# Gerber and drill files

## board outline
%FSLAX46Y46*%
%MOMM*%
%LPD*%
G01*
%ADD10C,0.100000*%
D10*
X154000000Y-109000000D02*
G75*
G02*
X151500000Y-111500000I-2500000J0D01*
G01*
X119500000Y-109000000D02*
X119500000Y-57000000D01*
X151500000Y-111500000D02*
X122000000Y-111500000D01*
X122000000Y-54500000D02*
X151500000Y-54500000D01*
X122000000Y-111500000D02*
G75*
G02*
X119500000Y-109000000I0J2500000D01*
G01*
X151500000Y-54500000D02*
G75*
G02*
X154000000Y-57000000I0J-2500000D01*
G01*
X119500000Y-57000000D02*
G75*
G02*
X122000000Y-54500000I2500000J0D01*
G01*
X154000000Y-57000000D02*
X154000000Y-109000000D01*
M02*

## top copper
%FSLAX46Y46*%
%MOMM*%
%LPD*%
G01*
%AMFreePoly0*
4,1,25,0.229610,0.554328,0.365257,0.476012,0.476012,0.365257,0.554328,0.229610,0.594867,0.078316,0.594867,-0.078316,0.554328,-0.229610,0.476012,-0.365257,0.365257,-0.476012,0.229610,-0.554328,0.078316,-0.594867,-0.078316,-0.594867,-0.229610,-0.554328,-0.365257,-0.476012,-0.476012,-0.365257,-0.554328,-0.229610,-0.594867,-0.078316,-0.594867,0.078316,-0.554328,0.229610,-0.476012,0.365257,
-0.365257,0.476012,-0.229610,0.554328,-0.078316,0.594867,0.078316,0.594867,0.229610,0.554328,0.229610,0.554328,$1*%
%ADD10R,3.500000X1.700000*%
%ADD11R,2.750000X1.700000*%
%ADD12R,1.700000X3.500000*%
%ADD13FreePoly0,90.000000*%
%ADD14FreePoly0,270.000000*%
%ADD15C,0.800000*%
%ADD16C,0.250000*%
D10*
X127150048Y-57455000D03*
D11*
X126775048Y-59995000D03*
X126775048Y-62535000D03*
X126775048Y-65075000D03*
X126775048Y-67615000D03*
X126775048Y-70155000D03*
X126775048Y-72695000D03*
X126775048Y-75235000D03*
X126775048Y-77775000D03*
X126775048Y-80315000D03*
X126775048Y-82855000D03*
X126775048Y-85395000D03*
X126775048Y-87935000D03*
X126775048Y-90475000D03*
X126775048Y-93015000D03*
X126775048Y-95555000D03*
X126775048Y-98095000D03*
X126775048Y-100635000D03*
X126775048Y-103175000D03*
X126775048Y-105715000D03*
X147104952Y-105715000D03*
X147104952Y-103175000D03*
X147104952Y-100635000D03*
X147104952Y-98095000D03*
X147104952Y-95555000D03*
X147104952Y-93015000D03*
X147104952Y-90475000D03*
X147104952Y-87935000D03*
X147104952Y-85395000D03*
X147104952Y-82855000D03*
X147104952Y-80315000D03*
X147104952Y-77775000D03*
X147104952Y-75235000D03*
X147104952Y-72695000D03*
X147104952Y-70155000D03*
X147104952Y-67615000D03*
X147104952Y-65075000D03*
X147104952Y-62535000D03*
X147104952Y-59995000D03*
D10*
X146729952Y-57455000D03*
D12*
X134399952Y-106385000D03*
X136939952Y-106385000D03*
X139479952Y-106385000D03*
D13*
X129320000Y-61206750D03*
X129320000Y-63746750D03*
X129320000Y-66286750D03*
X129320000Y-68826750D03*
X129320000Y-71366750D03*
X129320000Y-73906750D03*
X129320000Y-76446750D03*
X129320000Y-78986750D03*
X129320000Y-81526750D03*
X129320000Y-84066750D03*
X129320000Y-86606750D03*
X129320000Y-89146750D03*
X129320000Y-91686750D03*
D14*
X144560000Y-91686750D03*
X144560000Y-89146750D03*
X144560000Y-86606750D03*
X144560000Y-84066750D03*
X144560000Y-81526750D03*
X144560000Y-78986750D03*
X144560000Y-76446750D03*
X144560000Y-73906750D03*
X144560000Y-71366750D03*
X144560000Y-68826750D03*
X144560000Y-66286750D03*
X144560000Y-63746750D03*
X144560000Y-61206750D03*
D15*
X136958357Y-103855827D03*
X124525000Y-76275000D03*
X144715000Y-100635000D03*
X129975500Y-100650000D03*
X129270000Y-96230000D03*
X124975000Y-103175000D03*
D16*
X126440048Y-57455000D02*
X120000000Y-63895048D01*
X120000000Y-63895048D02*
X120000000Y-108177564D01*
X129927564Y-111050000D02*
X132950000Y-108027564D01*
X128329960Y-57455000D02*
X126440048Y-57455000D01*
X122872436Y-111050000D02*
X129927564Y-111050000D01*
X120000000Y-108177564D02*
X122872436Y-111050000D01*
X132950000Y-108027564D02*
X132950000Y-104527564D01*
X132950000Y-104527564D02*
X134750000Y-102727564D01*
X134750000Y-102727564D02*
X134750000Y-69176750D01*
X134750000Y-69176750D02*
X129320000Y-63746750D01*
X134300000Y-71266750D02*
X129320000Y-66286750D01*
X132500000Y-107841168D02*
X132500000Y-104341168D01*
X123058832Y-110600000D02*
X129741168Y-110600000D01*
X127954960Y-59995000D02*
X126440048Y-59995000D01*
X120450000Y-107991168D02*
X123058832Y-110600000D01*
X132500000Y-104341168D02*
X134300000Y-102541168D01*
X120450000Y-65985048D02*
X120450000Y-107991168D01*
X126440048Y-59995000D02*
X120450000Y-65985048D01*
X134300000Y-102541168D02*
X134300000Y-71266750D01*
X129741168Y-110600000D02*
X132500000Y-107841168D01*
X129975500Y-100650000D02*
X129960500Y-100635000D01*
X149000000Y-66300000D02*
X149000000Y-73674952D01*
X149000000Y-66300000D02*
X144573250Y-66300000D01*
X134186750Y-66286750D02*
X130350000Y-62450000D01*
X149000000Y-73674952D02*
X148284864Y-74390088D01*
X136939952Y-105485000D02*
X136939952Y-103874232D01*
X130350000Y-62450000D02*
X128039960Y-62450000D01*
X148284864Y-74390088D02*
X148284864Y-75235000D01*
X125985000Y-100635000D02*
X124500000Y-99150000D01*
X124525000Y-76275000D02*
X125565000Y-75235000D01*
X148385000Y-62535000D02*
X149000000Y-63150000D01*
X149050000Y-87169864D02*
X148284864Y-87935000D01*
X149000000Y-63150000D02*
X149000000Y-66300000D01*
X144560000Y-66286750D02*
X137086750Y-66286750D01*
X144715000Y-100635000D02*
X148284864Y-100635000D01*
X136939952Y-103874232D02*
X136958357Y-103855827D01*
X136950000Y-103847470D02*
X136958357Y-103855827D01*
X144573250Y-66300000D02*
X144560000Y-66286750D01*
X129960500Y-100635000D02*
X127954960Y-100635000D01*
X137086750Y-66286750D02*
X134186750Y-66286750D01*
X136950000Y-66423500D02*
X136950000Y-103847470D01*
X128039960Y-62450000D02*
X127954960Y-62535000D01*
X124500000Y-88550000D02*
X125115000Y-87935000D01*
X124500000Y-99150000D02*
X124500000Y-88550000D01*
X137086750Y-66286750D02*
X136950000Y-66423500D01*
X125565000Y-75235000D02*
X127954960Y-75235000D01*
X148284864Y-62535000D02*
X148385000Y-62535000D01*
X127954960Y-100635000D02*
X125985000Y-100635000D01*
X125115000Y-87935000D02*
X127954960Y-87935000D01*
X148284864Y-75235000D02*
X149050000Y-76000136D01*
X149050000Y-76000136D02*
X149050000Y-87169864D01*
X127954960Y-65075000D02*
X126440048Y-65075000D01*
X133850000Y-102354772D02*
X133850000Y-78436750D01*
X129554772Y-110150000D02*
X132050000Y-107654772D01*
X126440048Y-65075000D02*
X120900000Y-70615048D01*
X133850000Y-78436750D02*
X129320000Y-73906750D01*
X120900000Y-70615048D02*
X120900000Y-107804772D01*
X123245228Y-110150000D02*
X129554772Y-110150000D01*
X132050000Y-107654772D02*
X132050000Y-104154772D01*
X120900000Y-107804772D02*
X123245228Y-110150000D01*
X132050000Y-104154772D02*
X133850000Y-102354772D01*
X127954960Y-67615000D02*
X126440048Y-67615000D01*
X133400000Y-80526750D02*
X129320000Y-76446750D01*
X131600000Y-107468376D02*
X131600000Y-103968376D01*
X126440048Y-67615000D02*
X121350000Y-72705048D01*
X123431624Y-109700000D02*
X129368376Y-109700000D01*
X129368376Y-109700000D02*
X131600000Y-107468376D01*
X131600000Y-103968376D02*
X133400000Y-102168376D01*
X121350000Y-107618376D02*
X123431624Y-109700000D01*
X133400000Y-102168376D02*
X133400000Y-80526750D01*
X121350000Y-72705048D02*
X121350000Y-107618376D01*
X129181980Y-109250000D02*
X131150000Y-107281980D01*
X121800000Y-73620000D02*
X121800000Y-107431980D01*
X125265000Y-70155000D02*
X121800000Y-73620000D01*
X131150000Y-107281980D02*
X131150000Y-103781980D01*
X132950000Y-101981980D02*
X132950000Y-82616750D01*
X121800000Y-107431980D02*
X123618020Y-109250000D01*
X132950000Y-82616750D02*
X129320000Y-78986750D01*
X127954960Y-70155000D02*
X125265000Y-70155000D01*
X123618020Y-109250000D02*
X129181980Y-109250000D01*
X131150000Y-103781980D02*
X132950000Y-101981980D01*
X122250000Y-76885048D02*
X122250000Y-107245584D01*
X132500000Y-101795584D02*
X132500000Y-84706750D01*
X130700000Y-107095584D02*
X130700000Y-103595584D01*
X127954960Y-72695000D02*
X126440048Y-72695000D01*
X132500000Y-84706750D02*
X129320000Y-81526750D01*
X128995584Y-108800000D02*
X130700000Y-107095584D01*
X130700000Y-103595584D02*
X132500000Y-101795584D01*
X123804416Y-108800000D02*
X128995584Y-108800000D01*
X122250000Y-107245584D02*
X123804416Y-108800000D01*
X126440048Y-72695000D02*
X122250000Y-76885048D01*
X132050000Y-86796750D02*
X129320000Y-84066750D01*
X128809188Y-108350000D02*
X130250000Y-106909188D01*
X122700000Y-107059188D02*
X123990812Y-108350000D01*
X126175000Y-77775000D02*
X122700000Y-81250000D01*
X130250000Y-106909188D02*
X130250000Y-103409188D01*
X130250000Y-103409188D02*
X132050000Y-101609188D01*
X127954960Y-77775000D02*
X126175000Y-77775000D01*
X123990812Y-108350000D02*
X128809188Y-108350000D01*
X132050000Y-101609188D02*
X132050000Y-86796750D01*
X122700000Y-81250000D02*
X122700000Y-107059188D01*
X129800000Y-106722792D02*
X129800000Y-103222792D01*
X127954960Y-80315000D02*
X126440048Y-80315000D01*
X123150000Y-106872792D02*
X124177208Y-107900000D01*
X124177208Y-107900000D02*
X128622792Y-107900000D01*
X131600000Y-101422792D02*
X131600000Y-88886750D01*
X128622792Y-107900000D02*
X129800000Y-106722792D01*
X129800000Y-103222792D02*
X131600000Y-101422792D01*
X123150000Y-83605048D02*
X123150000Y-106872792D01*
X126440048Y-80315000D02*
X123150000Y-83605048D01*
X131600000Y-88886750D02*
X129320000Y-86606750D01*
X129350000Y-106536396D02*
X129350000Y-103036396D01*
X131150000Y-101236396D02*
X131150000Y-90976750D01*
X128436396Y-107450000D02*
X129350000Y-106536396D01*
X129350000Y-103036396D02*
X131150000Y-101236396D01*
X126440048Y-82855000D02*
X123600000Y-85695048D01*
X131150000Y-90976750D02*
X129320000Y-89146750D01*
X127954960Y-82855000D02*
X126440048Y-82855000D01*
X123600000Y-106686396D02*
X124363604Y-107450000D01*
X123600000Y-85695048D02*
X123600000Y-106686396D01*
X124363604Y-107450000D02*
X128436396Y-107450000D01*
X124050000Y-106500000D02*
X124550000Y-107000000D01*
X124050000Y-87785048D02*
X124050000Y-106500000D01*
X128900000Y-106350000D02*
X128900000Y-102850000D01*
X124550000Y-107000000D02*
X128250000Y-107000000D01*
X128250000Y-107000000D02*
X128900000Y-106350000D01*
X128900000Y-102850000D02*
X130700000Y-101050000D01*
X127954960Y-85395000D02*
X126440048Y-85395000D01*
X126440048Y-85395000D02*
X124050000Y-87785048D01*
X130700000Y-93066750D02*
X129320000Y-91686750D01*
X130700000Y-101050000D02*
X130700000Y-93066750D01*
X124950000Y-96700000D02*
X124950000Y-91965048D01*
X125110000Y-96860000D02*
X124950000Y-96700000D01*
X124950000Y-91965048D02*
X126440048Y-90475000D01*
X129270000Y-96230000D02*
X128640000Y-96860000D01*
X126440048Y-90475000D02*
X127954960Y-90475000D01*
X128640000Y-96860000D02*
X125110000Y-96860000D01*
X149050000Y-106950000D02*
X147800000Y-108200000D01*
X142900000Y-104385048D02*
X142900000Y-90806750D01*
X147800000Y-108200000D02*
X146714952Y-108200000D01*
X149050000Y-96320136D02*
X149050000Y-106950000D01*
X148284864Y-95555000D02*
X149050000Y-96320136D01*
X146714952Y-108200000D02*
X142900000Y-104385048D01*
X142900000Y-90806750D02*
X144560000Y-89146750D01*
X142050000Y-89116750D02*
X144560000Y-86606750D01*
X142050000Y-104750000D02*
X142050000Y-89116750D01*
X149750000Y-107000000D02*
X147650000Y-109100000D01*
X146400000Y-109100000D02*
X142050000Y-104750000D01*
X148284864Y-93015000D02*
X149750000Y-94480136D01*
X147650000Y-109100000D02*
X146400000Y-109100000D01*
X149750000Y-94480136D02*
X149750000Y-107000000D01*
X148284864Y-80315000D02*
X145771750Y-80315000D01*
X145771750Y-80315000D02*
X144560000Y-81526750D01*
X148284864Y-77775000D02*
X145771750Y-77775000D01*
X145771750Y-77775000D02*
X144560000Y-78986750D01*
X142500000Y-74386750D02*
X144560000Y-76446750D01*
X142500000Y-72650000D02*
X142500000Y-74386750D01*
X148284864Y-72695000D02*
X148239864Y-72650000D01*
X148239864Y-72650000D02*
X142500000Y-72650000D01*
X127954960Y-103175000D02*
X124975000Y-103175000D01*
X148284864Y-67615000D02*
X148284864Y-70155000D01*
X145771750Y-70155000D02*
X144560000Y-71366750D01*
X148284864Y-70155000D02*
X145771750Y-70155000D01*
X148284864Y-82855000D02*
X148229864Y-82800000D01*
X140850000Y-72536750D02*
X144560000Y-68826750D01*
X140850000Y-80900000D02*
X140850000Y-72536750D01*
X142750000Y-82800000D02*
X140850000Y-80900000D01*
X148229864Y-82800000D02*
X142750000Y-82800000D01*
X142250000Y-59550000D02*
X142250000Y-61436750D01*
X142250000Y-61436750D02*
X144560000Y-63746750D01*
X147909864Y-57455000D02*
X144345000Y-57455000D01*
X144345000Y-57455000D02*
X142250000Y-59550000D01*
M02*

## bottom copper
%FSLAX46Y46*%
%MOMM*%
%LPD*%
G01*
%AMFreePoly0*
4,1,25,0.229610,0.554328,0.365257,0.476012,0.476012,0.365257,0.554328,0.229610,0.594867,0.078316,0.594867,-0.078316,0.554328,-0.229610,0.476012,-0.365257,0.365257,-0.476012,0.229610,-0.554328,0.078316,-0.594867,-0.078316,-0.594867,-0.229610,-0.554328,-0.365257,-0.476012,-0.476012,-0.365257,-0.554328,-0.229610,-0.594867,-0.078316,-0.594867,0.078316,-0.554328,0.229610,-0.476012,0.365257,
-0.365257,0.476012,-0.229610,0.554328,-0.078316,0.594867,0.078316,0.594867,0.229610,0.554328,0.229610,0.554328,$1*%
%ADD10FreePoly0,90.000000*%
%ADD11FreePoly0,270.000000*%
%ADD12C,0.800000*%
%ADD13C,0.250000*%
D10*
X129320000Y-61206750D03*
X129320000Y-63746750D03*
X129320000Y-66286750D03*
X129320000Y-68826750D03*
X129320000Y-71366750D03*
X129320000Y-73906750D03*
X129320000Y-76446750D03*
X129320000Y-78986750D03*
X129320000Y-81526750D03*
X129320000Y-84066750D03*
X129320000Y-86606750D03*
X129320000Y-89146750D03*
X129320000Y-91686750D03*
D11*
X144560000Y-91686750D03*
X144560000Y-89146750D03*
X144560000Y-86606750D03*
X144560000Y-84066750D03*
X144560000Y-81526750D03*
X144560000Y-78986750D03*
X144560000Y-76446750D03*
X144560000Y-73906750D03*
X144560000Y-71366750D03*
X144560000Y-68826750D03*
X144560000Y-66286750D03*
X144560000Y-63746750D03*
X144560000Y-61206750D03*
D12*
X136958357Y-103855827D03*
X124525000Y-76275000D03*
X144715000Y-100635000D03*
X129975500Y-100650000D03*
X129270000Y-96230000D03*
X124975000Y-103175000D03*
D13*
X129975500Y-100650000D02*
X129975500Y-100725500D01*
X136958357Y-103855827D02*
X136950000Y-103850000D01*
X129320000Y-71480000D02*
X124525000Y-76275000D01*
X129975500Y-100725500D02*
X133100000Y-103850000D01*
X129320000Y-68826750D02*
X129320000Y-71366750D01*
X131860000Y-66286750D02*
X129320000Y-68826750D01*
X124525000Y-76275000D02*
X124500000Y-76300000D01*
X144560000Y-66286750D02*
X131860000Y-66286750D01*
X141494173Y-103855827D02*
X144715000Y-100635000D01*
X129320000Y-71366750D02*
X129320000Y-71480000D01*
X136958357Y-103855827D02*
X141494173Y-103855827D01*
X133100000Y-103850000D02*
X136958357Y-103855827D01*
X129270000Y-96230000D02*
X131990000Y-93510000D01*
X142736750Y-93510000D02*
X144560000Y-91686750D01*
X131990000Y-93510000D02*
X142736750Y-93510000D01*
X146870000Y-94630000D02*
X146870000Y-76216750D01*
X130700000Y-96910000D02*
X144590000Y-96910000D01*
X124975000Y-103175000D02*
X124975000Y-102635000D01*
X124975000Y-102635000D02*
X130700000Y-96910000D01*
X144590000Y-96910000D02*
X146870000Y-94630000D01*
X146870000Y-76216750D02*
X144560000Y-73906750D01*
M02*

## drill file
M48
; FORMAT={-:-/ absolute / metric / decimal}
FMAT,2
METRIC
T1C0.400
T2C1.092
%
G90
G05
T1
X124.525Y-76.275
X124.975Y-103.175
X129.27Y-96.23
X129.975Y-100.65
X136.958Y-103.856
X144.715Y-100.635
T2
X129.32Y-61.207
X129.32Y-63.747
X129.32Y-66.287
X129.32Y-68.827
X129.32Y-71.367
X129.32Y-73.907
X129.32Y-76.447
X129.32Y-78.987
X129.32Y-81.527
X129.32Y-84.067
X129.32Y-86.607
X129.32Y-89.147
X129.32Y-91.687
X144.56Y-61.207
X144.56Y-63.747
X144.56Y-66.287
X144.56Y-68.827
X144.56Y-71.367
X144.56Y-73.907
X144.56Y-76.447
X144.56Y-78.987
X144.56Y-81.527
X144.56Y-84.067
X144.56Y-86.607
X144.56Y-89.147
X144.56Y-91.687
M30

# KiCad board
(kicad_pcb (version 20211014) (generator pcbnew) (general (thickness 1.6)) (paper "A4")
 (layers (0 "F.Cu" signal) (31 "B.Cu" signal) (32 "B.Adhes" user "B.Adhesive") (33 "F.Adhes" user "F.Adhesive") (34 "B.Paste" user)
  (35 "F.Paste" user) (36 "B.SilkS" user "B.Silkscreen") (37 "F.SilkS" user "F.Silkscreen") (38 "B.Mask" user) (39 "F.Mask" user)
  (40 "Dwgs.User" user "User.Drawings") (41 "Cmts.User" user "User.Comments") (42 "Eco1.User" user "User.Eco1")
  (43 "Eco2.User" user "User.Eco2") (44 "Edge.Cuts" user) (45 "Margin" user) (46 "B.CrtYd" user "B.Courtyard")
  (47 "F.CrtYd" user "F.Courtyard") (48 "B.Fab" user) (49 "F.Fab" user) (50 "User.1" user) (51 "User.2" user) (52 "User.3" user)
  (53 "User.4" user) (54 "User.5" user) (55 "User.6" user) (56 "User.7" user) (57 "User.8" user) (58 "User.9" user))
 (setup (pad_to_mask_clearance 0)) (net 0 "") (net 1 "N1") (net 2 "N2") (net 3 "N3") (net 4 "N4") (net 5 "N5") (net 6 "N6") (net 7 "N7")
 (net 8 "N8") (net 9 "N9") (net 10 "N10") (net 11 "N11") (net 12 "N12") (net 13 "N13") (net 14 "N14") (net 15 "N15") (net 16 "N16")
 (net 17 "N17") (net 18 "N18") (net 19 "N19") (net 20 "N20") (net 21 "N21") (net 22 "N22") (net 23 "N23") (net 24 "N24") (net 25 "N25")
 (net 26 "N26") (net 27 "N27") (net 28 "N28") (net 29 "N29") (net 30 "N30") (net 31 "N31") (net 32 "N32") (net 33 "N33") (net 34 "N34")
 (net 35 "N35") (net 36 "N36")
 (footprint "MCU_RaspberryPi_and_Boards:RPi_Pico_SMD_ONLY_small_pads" (layer "F.Cu") (at 136.939952 81.585)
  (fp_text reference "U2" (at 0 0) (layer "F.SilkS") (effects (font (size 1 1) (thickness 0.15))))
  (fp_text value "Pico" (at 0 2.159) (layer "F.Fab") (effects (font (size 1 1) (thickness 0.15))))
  (pad "1" smd rect (at -8.609992 -24.13) (size 3.5 1.7) (drill (offset -1.179912 0)) (layers "F.Cu" "F.Mask") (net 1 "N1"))
  (pad "2" smd rect (at -8.984992 -21.59) (size 2.75 1.7) (drill (offset -1.179912 0)) (layers "F.Cu" "F.Mask") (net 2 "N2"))
  (pad "3" smd rect (at -8.984992 -19.05) (size 2.75 1.7) (drill (offset -1.179912 0)) (layers "F.Cu" "F.Mask") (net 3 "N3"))
  (pad "4" smd rect (at -8.984992 -16.51) (size 2.75 1.7) (drill (offset -1.179912 0)) (layers "F.Cu" "F.Mask") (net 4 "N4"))
  (pad "5" smd rect (at -8.984992 -13.97) (size 2.75 1.7) (drill (offset -1.179912 0)) (layers "F.Cu" "F.Mask") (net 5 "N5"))
  (pad "6" smd rect (at -8.984992 -11.43) (size 2.75 1.7) (drill (offset -1.179912 0)) (layers "F.Cu" "F.Mask") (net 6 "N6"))
  (pad "7" smd rect (at -8.984992 -8.89) (size 2.75 1.7) (drill (offset -1.179912 0)) (layers "F.Cu" "F.Mask") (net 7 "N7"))
  (pad "8" smd rect (at -8.984992 -6.35) (size 2.75 1.7) (drill (offset -1.179912 0)) (layers "F.Cu" "F.Mask") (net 3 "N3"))
  (pad "9" smd rect (at -8.984992 -3.81) (size 2.75 1.7) (drill (offset -1.179912 0)) (layers "F.Cu" "F.Mask") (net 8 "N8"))
  (pad "10" smd rect (at -8.984992 -1.27) (size 2.75 1.7) (drill (offset -1.179912 0)) (layers "F.Cu" "F.Mask") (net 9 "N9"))
  (pad "11" smd rect (at -8.984992 1.27) (size 2.75 1.7) (drill (offset -1.179912 0)) (layers "F.Cu" "F.Mask") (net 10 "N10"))
  (pad "12" smd rect (at -8.984992 3.81) (size 2.75 1.7) (drill (offset -1.179912 0)) (layers "F.Cu" "F.Mask") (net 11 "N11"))
  (pad "13" smd rect (at -8.984992 6.35) (size 2.75 1.7) (drill (offset -1.179912 0)) (layers "F.Cu" "F.Mask") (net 3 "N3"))
  (pad "14" smd rect (at -8.984992 8.89) (size 2.75 1.7) (drill (offset -1.179912 0)) (layers "F.Cu" "F.Mask") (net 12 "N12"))
  (pad "15" smd rect (at -8.984992 11.43) (size 2.75 1.7) (drill (offset -1.179912 0)) (layers "F.Cu" "F.Mask") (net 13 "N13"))
  (pad "16" smd rect (at -8.984992 13.97) (size 2.75 1.7) (drill (offset -1.179912 0)) (layers "F.Cu" "F.Mask") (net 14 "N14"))
  (pad "17" smd rect (at -8.984992 16.51) (size 2.75 1.7) (drill (offset -1.179912 0)) (layers "F.Cu" "F.Mask") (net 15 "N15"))
  (pad "18" smd rect (at -8.984992 19.05) (size 2.75 1.7) (drill (offset -1.179912 0)) (layers "F.Cu" "F.Mask") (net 3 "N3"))
  (pad "19" smd rect (at -8.984992 21.59) (size 2.75 1.7) (drill (offset -1.179912 0)) (layers "F.Cu" "F.Mask") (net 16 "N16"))
  (pad "20" smd rect (at -8.984992 24.13) (size 2.75 1.7) (drill (offset -1.179912 0)) (layers "F.Cu" "F.Mask") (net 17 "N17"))
  (pad "21" smd rect (at 11.344912 24.13) (size 2.75 1.7) (drill (offset -1.179912 0)) (layers "F.Cu" "F.Mask") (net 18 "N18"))
  (pad "22" smd rect (at 11.344912 21.59) (size 2.75 1.7) (drill (offset -1.179912 0)) (layers "F.Cu" "F.Mask") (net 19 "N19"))
  (pad "23" smd rect (at 11.344912 19.05) (size 2.75 1.7) (drill (offset -1.179912 0)) (layers "F.Cu" "F.Mask") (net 3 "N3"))
  (pad "24" smd rect (at 11.344912 16.51) (size 2.75 1.7) (drill (offset -1.179912 0)) (layers "F.Cu" "F.Mask") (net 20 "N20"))
  (pad "25" smd rect (at 11.344912 13.97) (size 2.75 1.7) (drill (offset -1.179912 0)) (layers "F.Cu" "F.Mask") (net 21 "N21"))
  (pad "26" smd rect (at 11.344912 11.43) (size 2.75 1.7) (drill (offset -1.179912 0)) (layers "F.Cu" "F.Mask") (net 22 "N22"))
  (pad "27" smd rect (at 11.344912 8.89) (size 2.75 1.7) (drill (offset -1.179912 0)) (layers "F.Cu" "F.Mask") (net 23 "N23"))
  (pad "28" smd rect (at 11.344912 6.35) (size 2.75 1.7) (drill (offset -1.179912 0)) (layers "F.Cu" "F.Mask") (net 3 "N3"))
  (pad "29" smd rect (at 11.344912 3.81) (size 2.75 1.7) (drill (offset -1.179912 0)) (layers "F.Cu" "F.Mask") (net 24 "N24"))
  (pad "30" smd rect (at 11.344912 1.27) (size 2.75 1.7) (drill (offset -1.179912 0)) (layers "F.Cu" "F.Mask") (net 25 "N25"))
  (pad "31" smd rect (at 11.344912 -1.27) (size 2.75 1.7) (drill (offset -1.179912 0)) (layers "F.Cu" "F.Mask") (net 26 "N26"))
  (pad "32" smd rect (at 11.344912 -3.81) (size 2.75 1.7) (drill (offset -1.179912 0)) (layers "F.Cu" "F.Mask") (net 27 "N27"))
  (pad "33" smd rect (at 11.344912 -6.35) (size 2.75 1.7) (drill (offset -1.179912 0)) (layers "F.Cu" "F.Mask") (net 3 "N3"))
  (pad "34" smd rect (at 11.344912 -8.89) (size 2.75 1.7) (drill (offset -1.179912 0)) (layers "F.Cu" "F.Mask") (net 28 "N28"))
  (pad "35" smd rect (at 11.344912 -11.43) (size 2.75 1.7) (drill (offset -1.179912 0)) (layers "F.Cu" "F.Mask") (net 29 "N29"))
  (pad "36" smd rect (at 11.344912 -13.97) (size 2.75 1.7) (drill (offset -1.179912 0)) (layers "F.Cu" "F.Mask") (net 29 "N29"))
  (pad "37" smd rect (at 11.344912 -16.51) (size 2.75 1.7) (drill (offset -1.179912 0)) (layers "F.Cu" "F.Mask") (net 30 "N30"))
  (pad "38" smd rect (at 11.344912 -19.05) (size 2.75 1.7) (drill (offset -1.179912 0)) (layers "F.Cu" "F.Mask") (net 3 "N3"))
  (pad "39" smd rect (at 11.344912 -21.59) (size 2.75 1.7) (drill (offset -1.179912 0)) (layers "F.Cu" "F.Mask") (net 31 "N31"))
  (pad "40" smd rect (at 10.969912 -24.13) (size 3.5 1.7) (drill (offset -1.179912 0)) (layers "F.Cu" "F.Mask") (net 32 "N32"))
  (pad "41" smd rect (at -2.54 23.9 90) (size 3.5 1.7) (drill (offset -0.9 0)) (layers "F.Cu" "F.Mask") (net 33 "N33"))
  (pad "42" smd rect (at 0 23.9 90) (size 3.5 1.7) (drill (offset -0.9 0)) (layers "F.Cu" "F.Mask") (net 3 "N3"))
  (pad "43" smd rect (at 2.54 23.9 90) (size 3.5 1.7) (drill (offset -0.9 0)) (layers "F.Cu" "F.Mask") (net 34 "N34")))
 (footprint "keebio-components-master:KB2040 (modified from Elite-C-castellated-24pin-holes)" (layer "B.Cu") (at 136.94 77.71675 -90)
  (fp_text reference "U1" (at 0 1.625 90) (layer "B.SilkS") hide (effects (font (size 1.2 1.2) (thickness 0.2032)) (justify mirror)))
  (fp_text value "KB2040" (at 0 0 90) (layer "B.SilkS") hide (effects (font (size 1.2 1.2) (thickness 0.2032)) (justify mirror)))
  (pad "0" thru_hole custom (at -16.51 7.62 90) (size 1.2 1.2) (drill 1.0922) (layers *.Cu *.SilkS *.Mask) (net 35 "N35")
   (options (clearance outline) (anchor circle)) (primitives))
  (pad "1" thru_hole custom (at -13.97 7.62 90) (size 1.2 1.2) (drill 1.0922) (layers *.Cu *.SilkS *.Mask) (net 1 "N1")
   (options (clearance outline) (anchor circle)) (primitives))
  (pad "2" thru_hole custom (at -11.43 7.62 90) (size 1.2 1.2) (drill 1.0922) (layers *.Cu *.SilkS *.Mask) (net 2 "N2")
   (options (clearance outline) (anchor circle)) (primitives))
  (pad "3" thru_hole custom (at -8.89 7.62 90) (size 1.2 1.2) (drill 1.0922) (layers *.Cu *.SilkS *.Mask) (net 3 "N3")
   (options (clearance outline) (anchor circle)) (primitives))
  (pad "4" thru_hole custom (at -6.35 7.62 90) (size 1.2 1.2) (drill 1.0922) (layers *.Cu *.SilkS *.Mask) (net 3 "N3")
   (options (clearance outline) (anchor circle)) (primitives))
  (pad "5" thru_hole custom (at -3.81 7.62 90) (size 1.2 1.2) (drill 1.0922) (layers *.Cu *.SilkS *.Mask) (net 4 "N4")
   (options (clearance outline) (anchor circle)) (primitives))
  (pad "6" thru_hole custom (at -1.27 7.62 90) (size 1.2 1.2) (drill 1.0922) (layers *.Cu *.SilkS *.Mask) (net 5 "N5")
   (options (clearance outline) (anchor circle)) (primitives))
  (pad "7" thru_hole custom (at 1.27 7.62 90) (size 1.2 1.2) (drill 1.0922) (layers *.Cu *.SilkS *.Mask) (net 6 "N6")
   (options (clearance outline) (anchor circle)) (primitives))
  (pad "8" thru_hole custom (at 3.81 7.62 90) (size 1.2 1.2) (drill 1.0922) (layers *.Cu *.SilkS *.Mask) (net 7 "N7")
   (options (clearance outline) (anchor circle)) (primitives))
  (pad "9" thru_hole custom (at 6.35 7.62 90) (size 1.2 1.2) (drill 1.0922) (layers *.Cu *.SilkS *.Mask) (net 8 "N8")
   (options (clearance outline) (anchor circle)) (primitives))
  (pad "10" thru_hole custom (at 8.89 7.62 90) (size 1.2 1.2) (drill 1.0922) (layers *.Cu *.SilkS *.Mask) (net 9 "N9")
   (options (clearance outline) (anchor circle)) (primitives))
  (pad "11" thru_hole custom (at 11.43 7.62 90) (size 1.2 1.2) (drill 1.0922) (layers *.Cu *.SilkS *.Mask) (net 10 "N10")
   (options (clearance outline) (anchor circle)) (primitives))
  (pad "12" thru_hole custom (at 13.97 7.62 90) (size 1.2 1.2) (drill 1.0922) (layers *.Cu *.SilkS *.Mask) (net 11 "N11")
   (options (clearance outline) (anchor circle)) (primitives))
  (pad "13" thru_hole custom (at 13.97 -7.62 270) (size 1.2 1.2) (drill 1.0922) (layers *.Cu *.SilkS *.Mask) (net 12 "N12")
   (options (clearance outline) (anchor circle)) (primitives))
  (pad "14" thru_hole custom (at 11.43 -7.62 270) (size 1.2 1.2) (drill 1.0922) (layers *.Cu *.SilkS *.Mask) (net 21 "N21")
   (options (clearance outline) (anchor circle)) (primitives))
  (pad "15" thru_hole custom (at 8.89 -7.62 270) (size 1.2 1.2) (drill 1.0922) (layers *.Cu *.SilkS *.Mask) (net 22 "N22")
   (options (clearance outline) (anchor circle)) (primitives))
  (pad "16" thru_hole custom (at 6.35 -7.62 270) (size 1.2 1.2) (drill 1.0922) (layers *.Cu *.SilkS *.Mask) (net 20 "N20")
   (options (clearance outline) (anchor circle)) (primitives))
  (pad "17" thru_hole custom (at 3.81 -7.62 270) (size 1.2 1.2) (drill 1.0922) (layers *.Cu *.SilkS *.Mask) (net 26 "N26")
   (options (clearance outline) (anchor circle)) (primitives))
  (pad "18" thru_hole custom (at 1.27 -7.62 270) (size 1.2 1.2) (drill 1.0922) (layers *.Cu *.SilkS *.Mask) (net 27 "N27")
   (options (clearance outline) (anchor circle)) (primitives))
  (pad "19" thru_hole custom (at -1.27 -7.62 270) (size 1.2 1.2) (drill 1.0922) (layers *.Cu *.SilkS *.Mask) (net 28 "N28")
   (options (clearance outline) (anchor circle)) (primitives))
  (pad "20" thru_hole custom (at -3.81 -7.62 270) (size 1.2 1.2) (drill 1.0922) (layers *.Cu *.SilkS *.Mask) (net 16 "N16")
   (options (clearance outline) (anchor circle)) (primitives))
  (pad "21" thru_hole custom (at -6.35 -7.62 270) (size 1.2 1.2) (drill 1.0922) (layers *.Cu *.SilkS *.Mask) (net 29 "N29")
   (options (clearance outline) (anchor circle)) (primitives))
  (pad "22" thru_hole custom (at -8.89 -7.62 270) (size 1.2 1.2) (drill 1.0922) (layers *.Cu *.SilkS *.Mask) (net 25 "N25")
   (options (clearance outline) (anchor circle)) (primitives))
  (pad "23" thru_hole custom (at -11.43 -7.62 270) (size 1.2 1.2) (drill 1.0922) (layers *.Cu *.SilkS *.Mask) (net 3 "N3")
   (options (clearance outline) (anchor circle)) (primitives))
  (pad "24" thru_hole custom (at -13.97 -7.62 270) (size 1.2 1.2) (drill 1.0922) (layers *.Cu *.SilkS *.Mask) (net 32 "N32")
   (options (clearance outline) (anchor circle)) (primitives))
  (pad "25" thru_hole custom (at -16.51 -7.62 270) (size 1.2 1.2) (drill 1.0922) (layers *.Cu *.SilkS *.Mask) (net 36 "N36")
   (options (clearance outline) (anchor circle)) (primitives)))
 (gr_arc (start 154 109) (mid 153.267767 110.767767) (end 151.5 111.5) (layer "Edge.Cuts") (width 0.1))
 (gr_line (start 119.5 109) (end 119.5 57) (layer "Edge.Cuts") (width 0.1))
 (gr_line (start 151.5 111.5) (end 122 111.5) (layer "Edge.Cuts") (width 0.1))
 (gr_line (start 122 54.5) (end 151.5 54.5) (layer "Edge.Cuts") (width 0.1))
 (gr_arc (start 122 111.5) (mid 120.232233 110.767767) (end 119.5 109) (layer "Edge.Cuts") (width 0.1))
 (gr_arc (start 151.5 54.5) (mid 153.267767 55.232233) (end 154 57) (layer "Edge.Cuts") (width 0.1))
 (gr_arc (start 119.5 57) (mid 120.232233 55.232233) (end 122 54.5) (layer "Edge.Cuts") (width 0.1))
 (gr_line (start 154 57) (end 154 109) (layer "Edge.Cuts") (width 0.1))
 (segment (start 126.440048 57.455) (end 120 63.895048) (width 0.25) (layer "F.Cu") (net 1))
 (segment (start 120 63.895048) (end 120 108.177564) (width 0.25) (layer "F.Cu") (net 1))
 (segment (start 129.927564 111.05) (end 132.95 108.027564) (width 0.25) (layer "F.Cu") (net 1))
 (segment (start 128.32996 57.455) (end 126.440048 57.455) (width 0.25) (layer "F.Cu") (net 1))
 (segment (start 122.872436 111.05) (end 129.927564 111.05) (width 0.25) (layer "F.Cu") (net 1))
 (segment (start 120 108.177564) (end 122.872436 111.05) (width 0.25) (layer "F.Cu") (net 1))
 (segment (start 132.95 108.027564) (end 132.95 104.527564) (width 0.25) (layer "F.Cu") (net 1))
 (segment (start 132.95 104.527564) (end 134.75 102.727564) (width 0.25) (layer "F.Cu") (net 1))
 (segment (start 134.75 102.727564) (end 134.75 69.17675) (width 0.25) (layer "F.Cu") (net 1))
 (segment (start 134.75 69.17675) (end 129.32 63.74675) (width 0.25) (layer "F.Cu") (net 1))
 (segment (start 134.3 71.26675) (end 129.32 66.28675) (width 0.25) (layer "F.Cu") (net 2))
 (segment (start 132.5 107.841168) (end 132.5 104.341168) (width 0.25) (layer "F.Cu") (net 2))
 (segment (start 123.058832 110.6) (end 129.741168 110.6) (width 0.25) (layer "F.Cu") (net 2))
 (segment (start 127.95496 59.995) (end 126.440048 59.995) (width 0.25) (layer "F.Cu") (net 2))
 (segment (start 120.45 107.991168) (end 123.058832 110.6) (width 0.25) (layer "F.Cu") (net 2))
 (segment (start 132.5 104.341168) (end 134.3 102.541168) (width 0.25) (layer "F.Cu") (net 2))
 (segment (start 120.45 65.985048) (end 120.45 107.991168) (width 0.25) (layer "F.Cu") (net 2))
 (segment (start 126.440048 59.995) (end 120.45 65.985048) (width 0.25) (layer "F.Cu") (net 2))
 (segment (start 134.3 102.541168) (end 134.3 71.26675) (width 0.25) (layer "F.Cu") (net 2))
 (segment (start 129.741168 110.6) (end 132.5 107.841168) (width 0.25) (layer "F.Cu") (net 2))
 (segment (start 129.9755 100.65) (end 129.9605 100.635) (width 0.25) (layer "F.Cu") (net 3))
 (segment (start 149 66.3) (end 149 73.674952) (width 0.25) (layer "F.Cu") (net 3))
 (segment (start 149 66.3) (end 144.57325 66.3) (width 0.25) (layer "F.Cu") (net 3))
 (segment (start 134.18675 66.28675) (end 130.35 62.45) (width 0.25) (layer "F.Cu") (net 3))
 (segment (start 149 73.674952) (end 148.284864 74.390088) (width 0.25) (layer "F.Cu") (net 3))
 (segment (start 136.939952 105.485) (end 136.939952 103.874232) (width 0.25) (layer "F.Cu") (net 3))
 (segment (start 130.35 62.45) (end 128.03996 62.45) (width 0.25) (layer "F.Cu") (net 3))
 (segment (start 148.284864 74.390088) (end 148.284864 75.235) (width 0.25) (layer "F.Cu") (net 3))
 (segment (start 125.985 100.635) (end 124.5 99.15) (width 0.25) (layer "F.Cu") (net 3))
 (segment (start 124.525 76.275) (end 125.565 75.235) (width 0.25) (layer "F.Cu") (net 3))
 (segment (start 148.385 62.535) (end 149 63.15) (width 0.25) (layer "F.Cu") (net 3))
 (segment (start 149.05 87.169864) (end 148.284864 87.935) (width 0.25) (layer "F.Cu") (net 3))
 (segment (start 149 63.15) (end 149 66.3) (width 0.25) (layer "F.Cu") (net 3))
 (segment (start 144.56 66.28675) (end 137.08675 66.28675) (width 0.25) (layer "F.Cu") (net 3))
 (segment (start 144.715 100.635) (end 148.284864 100.635) (width 0.25) (layer "F.Cu") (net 3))
 (segment (start 136.939952 103.874232) (end 136.958357 103.855827) (width 0.25) (layer "F.Cu") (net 3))
 (segment (start 136.95 103.84747) (end 136.958357 103.855827) (width 0.25) (layer "F.Cu") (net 3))
 (segment (start 144.57325 66.3) (end 144.56 66.28675) (width 0.25) (layer "F.Cu") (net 3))
 (segment (start 129.9605 100.635) (end 127.95496 100.635) (width 0.25) (layer "F.Cu") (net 3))
 (segment (start 137.08675 66.28675) (end 134.18675 66.28675) (width 0.25) (layer "F.Cu") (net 3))
 (segment (start 136.95 66.4235) (end 136.95 103.84747) (width 0.25) (layer "F.Cu") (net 3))
 (segment (start 128.03996 62.45) (end 127.95496 62.535) (width 0.25) (layer "F.Cu") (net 3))
 (segment (start 124.5 88.55) (end 125.115 87.935) (width 0.25) (layer "F.Cu") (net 3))
 (segment (start 124.5 99.15) (end 124.5 88.55) (width 0.25) (layer "F.Cu") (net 3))
 (segment (start 137.08675 66.28675) (end 136.95 66.4235) (width 0.25) (layer "F.Cu") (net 3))
 (segment (start 125.565 75.235) (end 127.95496 75.235) (width 0.25) (layer "F.Cu") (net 3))
 (segment (start 148.284864 62.535) (end 148.385 62.535) (width 0.25) (layer "F.Cu") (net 3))
 (segment (start 127.95496 100.635) (end 125.985 100.635) (width 0.25) (layer "F.Cu") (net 3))
 (segment (start 125.115 87.935) (end 127.95496 87.935) (width 0.25) (layer "F.Cu") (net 3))
 (segment (start 148.284864 75.235) (end 149.05 76.000136) (width 0.25) (layer "F.Cu") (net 3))
 (segment (start 149.05 76.000136) (end 149.05 87.169864) (width 0.25) (layer "F.Cu") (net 3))
 (via (at 136.958357 103.855827) (size 0.8) (drill 0.4) (layers "F.Cu" "B.Cu") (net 3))
 (via (at 124.525 76.275) (size 0.8) (drill 0.4) (layers "F.Cu" "B.Cu") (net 3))
 (via (at 144.715 100.635) (size 0.8) (drill 0.4) (layers "F.Cu" "B.Cu") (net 3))
 (via (at 129.9755 100.65) (size 0.8) (drill 0.4) (layers "F.Cu" "B.Cu") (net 3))
 (segment (start 129.9755 100.65) (end 129.9755 100.7255) (width 0.25) (layer "B.Cu") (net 3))
 (segment (start 136.958357 103.855827) (end 136.95 103.85) (width 0.25) (layer "B.Cu") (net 3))
 (segment (start 129.32 71.48) (end 124.525 76.275) (width 0.25) (layer "B.Cu") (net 3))
 (segment (start 129.9755 100.7255) (end 133.1 103.85) (width 0.25) (layer "B.Cu") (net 3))
 (segment (start 129.32 68.82675) (end 129.32 71.36675) (width 0.25) (layer "B.Cu") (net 3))
 (segment (start 131.86 66.28675) (end 129.32 68.82675) (width 0.25) (layer "B.Cu") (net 3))
 (segment (start 124.525 76.275) (end 124.5 76.3) (width 0.25) (layer "B.Cu") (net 3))
 (segment (start 144.56 66.28675) (end 131.86 66.28675) (width 0.25) (layer "B.Cu") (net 3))
 (segment (start 141.494173 103.855827) (end 144.715 100.635) (width 0.25) (layer "B.Cu") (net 3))
 (segment (start 129.32 71.36675) (end 129.32 71.48) (width 0.25) (layer "B.Cu") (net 3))
 (segment (start 136.958357 103.855827) (end 141.494173 103.855827) (width 0.25) (layer "B.Cu") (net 3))
 (segment (start 133.1 103.85) (end 136.958357 103.855827) (width 0.25) (layer "B.Cu") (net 3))
 (segment (start 127.95496 65.075) (end 126.440048 65.075) (width 0.25) (layer "F.Cu") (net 4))
 (segment (start 133.85 102.354772) (end 133.85 78.43675) (width 0.25) (layer "F.Cu") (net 4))
 (segment (start 129.554772 110.15) (end 132.05 107.654772) (width 0.25) (layer "F.Cu") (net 4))
 (segment (start 126.440048 65.075) (end 120.9 70.615048) (width 0.25) (layer "F.Cu") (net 4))
 (segment (start 133.85 78.43675) (end 129.32 73.90675) (width 0.25) (layer "F.Cu") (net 4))
 (segment (start 120.9 70.615048) (end 120.9 107.804772) (width 0.25) (layer "F.Cu") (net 4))
 (segment (start 123.245228 110.15) (end 129.554772 110.15) (width 0.25) (layer "F.Cu") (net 4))
 (segment (start 132.05 107.654772) (end 132.05 104.154772) (width 0.25) (layer "F.Cu") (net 4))
 (segment (start 120.9 107.804772) (end 123.245228 110.15) (width 0.25) (layer "F.Cu") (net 4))
 (segment (start 132.05 104.154772) (end 133.85 102.354772) (width 0.25) (layer "F.Cu") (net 4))
 (segment (start 127.95496 67.615) (end 126.440048 67.615) (width 0.25) (layer "F.Cu") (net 5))
 (segment (start 133.4 80.52675) (end 129.32 76.44675) (width 0.25) (layer "F.Cu") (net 5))
 (segment (start 131.6 107.468376) (end 131.6 103.968376) (width 0.25) (layer "F.Cu") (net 5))
 (segment (start 126.440048 67.615) (end 121.35 72.705048) (width 0.25) (layer "F.Cu") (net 5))
 (segment (start 123.431624 109.7) (end 129.368376 109.7) (width 0.25) (layer "F.Cu") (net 5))
 (segment (start 129.368376 109.7) (end 131.6 107.468376) (width 0.25) (layer "F.Cu") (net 5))
 (segment (start 131.6 103.968376) (end 133.4 102.168376) (width 0.25) (layer "F.Cu") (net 5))
 (segment (start 121.35 107.618376) (end 123.431624 109.7) (width 0.25) (layer "F.Cu") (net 5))
 (segment (start 133.4 102.168376) (end 133.4 80.52675) (width 0.25) (layer "F.Cu") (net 5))
 (segment (start 121.35 72.705048) (end 121.35 107.618376) (width 0.25) (layer "F.Cu") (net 5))
 (segment (start 129.18198 109.25) (end 131.15 107.28198) (width 0.25) (layer "F.Cu") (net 6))
 (segment (start 121.8 73.62) (end 121.8 107.43198) (width 0.25) (layer "F.Cu") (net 6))
 (segment (start 125.265 70.155) (end 121.8 73.62) (width 0.25) (layer "F.Cu") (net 6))
 (segment (start 131.15 107.28198) (end 131.15 103.78198) (width 0.25) (layer "F.Cu") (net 6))
 (segment (start 132.95 101.98198) (end 132.95 82.61675) (width 0.25) (layer "F.Cu") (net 6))
 (segment (start 121.8 107.43198) (end 123.61802 109.25) (width 0.25) (layer "F.Cu") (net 6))
 (segment (start 132.95 82.61675) (end 129.32 78.98675) (width 0.25) (layer "F.Cu") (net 6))
 (segment (start 127.95496 70.155) (end 125.265 70.155) (width 0.25) (layer "F.Cu") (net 6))
 (segment (start 123.61802 109.25) (end 129.18198 109.25) (width 0.25) (layer "F.Cu") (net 6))
 (segment (start 131.15 103.78198) (end 132.95 101.98198) (width 0.25) (layer "F.Cu") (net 6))
 (segment (start 122.25 76.885048) (end 122.25 107.245584) (width 0.25) (layer "F.Cu") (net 7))
 (segment (start 132.5 101.795584) (end 132.5 84.70675) (width 0.25) (layer "F.Cu") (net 7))
 (segment (start 130.7 107.095584) (end 130.7 103.595584) (width 0.25) (layer "F.Cu") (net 7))
 (segment (start 127.95496 72.695) (end 126.440048 72.695) (width 0.25) (layer "F.Cu") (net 7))
 (segment (start 132.5 84.70675) (end 129.32 81.52675) (width 0.25) (layer "F.Cu") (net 7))
 (segment (start 128.995584 108.8) (end 130.7 107.095584) (width 0.25) (layer "F.Cu") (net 7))
 (segment (start 130.7 103.595584) (end 132.5 101.795584) (width 0.25) (layer "F.Cu") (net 7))
 (segment (start 123.804416 108.8) (end 128.995584 108.8) (width 0.25) (layer "F.Cu") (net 7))
 (segment (start 122.25 107.245584) (end 123.804416 108.8) (width 0.25) (layer "F.Cu") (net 7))
 (segment (start 126.440048 72.695) (end 122.25 76.885048) (width 0.25) (layer "F.Cu") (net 7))
 (segment (start 132.05 86.79675) (end 129.32 84.06675) (width 0.25) (layer "F.Cu") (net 8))
 (segment (start 128.809188 108.35) (end 130.25 106.909188) (width 0.25) (layer "F.Cu") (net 8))
 (segment (start 122.7 107.059188) (end 123.990812 108.35) (width 0.25) (layer "F.Cu") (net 8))
 (segment (start 126.175 77.775) (end 122.7 81.25) (width 0.25) (layer "F.Cu") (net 8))
 (segment (start 130.25 106.909188) (end 130.25 103.409188) (width 0.25) (layer "F.Cu") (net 8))
 (segment (start 130.25 103.409188) (end 132.05 101.609188) (width 0.25) (layer "F.Cu") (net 8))
 (segment (start 127.95496 77.775) (end 126.175 77.775) (width 0.25) (layer "F.Cu") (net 8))
 (segment (start 123.990812 108.35) (end 128.809188 108.35) (width 0.25) (layer "F.Cu") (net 8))
 (segment (start 132.05 101.609188) (end 132.05 86.79675) (width 0.25) (layer "F.Cu") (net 8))
 (segment (start 122.7 81.25) (end 122.7 107.059188) (width 0.25) (layer "F.Cu") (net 8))
 (segment (start 129.8 106.722792) (end 129.8 103.222792) (width 0.25) (layer "F.Cu") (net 9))
 (segment (start 127.95496 80.315) (end 126.440048 80.315) (width 0.25) (layer "F.Cu") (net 9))
 (segment (start 123.15 106.872792) (end 124.177208 107.9) (width 0.25) (layer "F.Cu") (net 9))
 (segment (start 124.177208 107.9) (end 128.622792 107.9) (width 0.25) (layer "F.Cu") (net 9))
 (segment (start 131.6 101.422792) (end 131.6 88.88675) (width 0.25) (layer "F.Cu") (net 9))
 (segment (start 128.622792 107.9) (end 129.8 106.722792) (width 0.25) (layer "F.Cu") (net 9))
 (segment (start 129.8 103.222792) (end 131.6 101.422792) (width 0.25) (layer "F.Cu") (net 9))
 (segment (start 123.15 83.605048) (end 123.15 106.872792) (width 0.25) (layer "F.Cu") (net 9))
 (segment (start 126.440048 80.315) (end 123.15 83.605048) (width 0.25) (layer "F.Cu") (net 9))
 (segment (start 131.6 88.88675) (end 129.32 86.60675) (width 0.25) (layer "F.Cu") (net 9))
 (segment (start 129.35 106.536396) (end 129.35 103.036396) (width 0.25) (layer "F.Cu") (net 10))
 (segment (start 131.15 101.236396) (end 131.15 90.97675) (width 0.25) (layer "F.Cu") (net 10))
 (segment (start 128.436396 107.45) (end 129.35 106.536396) (width 0.25) (layer "F.Cu") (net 10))
 (segment (start 129.35 103.036396) (end 131.15 101.236396) (width 0.25) (layer "F.Cu") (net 10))
 (segment (start 126.440048 82.855) (end 123.6 85.695048) (width 0.25) (layer "F.Cu") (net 10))
 (segment (start 131.15 90.97675) (end 129.32 89.14675) (width 0.25) (layer "F.Cu") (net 10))
 (segment (start 127.95496 82.855) (end 126.440048 82.855) (width 0.25) (layer "F.Cu") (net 10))
 (segment (start 123.6 106.686396) (end 124.363604 107.45) (width 0.25) (layer "F.Cu") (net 10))
 (segment (start 123.6 85.695048) (end 123.6 106.686396) (width 0.25) (layer "F.Cu") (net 10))
 (segment (start 124.363604 107.45) (end 128.436396 107.45) (width 0.25) (layer "F.Cu") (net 10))
 (segment (start 124.05 106.5) (end 124.55 107) (width 0.25) (layer "F.Cu") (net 11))
 (segment (start 124.05 87.785048) (end 124.05 106.5) (width 0.25) (layer "F.Cu") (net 11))
 (segment (start 128.9 106.35) (end 128.9 102.85) (width 0.25) (layer "F.Cu") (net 11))
 (segment (start 124.55 107) (end 128.25 107) (width 0.25) (layer "F.Cu") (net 11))
 (segment (start 128.25 107) (end 128.9 106.35) (width 0.25) (layer "F.Cu") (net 11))
 (segment (start 128.9 102.85) (end 130.7 101.05) (width 0.25) (layer "F.Cu") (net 11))
 (segment (start 127.95496 85.395) (end 126.440048 85.395) (width 0.25) (layer "F.Cu") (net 11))
 (segment (start 126.440048 85.395) (end 124.05 87.785048) (width 0.25) (layer "F.Cu") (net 11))
 (segment (start 130.7 93.06675) (end 129.32 91.68675) (width 0.25) (layer "F.Cu") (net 11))
 (segment (start 130.7 101.05) (end 130.7 93.06675) (width 0.25) (layer "F.Cu") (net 11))
 (segment (start 124.95 96.7) (end 124.95 91.965048) (width 0.25) (layer "F.Cu") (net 12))
 (segment (start 125.11 96.86) (end 124.95 96.7) (width 0.25) (layer "F.Cu") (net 12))
 (segment (start 124.95 91.965048) (end 126.440048 90.475) (width 0.25) (layer "F.Cu") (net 12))
 (segment (start 129.27 96.23) (end 128.64 96.86) (width 0.25) (layer "F.Cu") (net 12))
 (segment (start 126.440048 90.475) (end 127.95496 90.475) (width 0.25) (layer "F.Cu") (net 12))
 (segment (start 128.64 96.86) (end 125.11 96.86) (width 0.25) (layer "F.Cu") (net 12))
 (via (at 129.27 96.23) (size 0.8) (drill 0.4) (layers "F.Cu" "B.Cu") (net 12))
 (segment (start 129.27 96.23) (end 131.99 93.51) (width 0.25) (layer "B.Cu") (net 12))
 (segment (start 142.73675 93.51) (end 144.56 91.68675) (width 0.25) (layer "B.Cu") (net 12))
 (segment (start 131.99 93.51) (end 142.73675 93.51) (width 0.25) (layer "B.Cu") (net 12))
 (segment (start 149.05 106.95) (end 147.8 108.2) (width 0.25) (layer "F.Cu") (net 21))
 (segment (start 142.9 104.385048) (end 142.9 90.80675) (width 0.25) (layer "F.Cu") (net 21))
 (segment (start 147.8 108.2) (end 146.714952 108.2) (width 0.25) (layer "F.Cu") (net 21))
 (segment (start 149.05 96.320136) (end 149.05 106.95) (width 0.25) (layer "F.Cu") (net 21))
 (segment (start 148.284864 95.555) (end 149.05 96.320136) (width 0.25) (layer "F.Cu") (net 21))
 (segment (start 146.714952 108.2) (end 142.9 104.385048) (width 0.25) (layer "F.Cu") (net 21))
 (segment (start 142.9 90.80675) (end 144.56 89.14675) (width 0.25) (layer "F.Cu") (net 21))
 (segment (start 142.05 89.11675) (end 144.56 86.60675) (width 0.25) (layer "F.Cu") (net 22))
 (segment (start 142.05 104.75) (end 142.05 89.11675) (width 0.25) (layer "F.Cu") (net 22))
 (segment (start 149.75 107) (end 147.65 109.1) (width 0.25) (layer "F.Cu") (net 22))
 (segment (start 146.4 109.1) (end 142.05 104.75) (width 0.25) (layer "F.Cu") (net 22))
 (segment (start 148.284864 93.015) (end 149.75 94.480136) (width 0.25) (layer "F.Cu") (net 22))
 (segment (start 147.65 109.1) (end 146.4 109.1) (width 0.25) (layer "F.Cu") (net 22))
 (segment (start 149.75 94.480136) (end 149.75 107) (width 0.25) (layer "F.Cu") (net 22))
 (segment (start 148.284864 80.315) (end 145.77175 80.315) (width 0.25) (layer "F.Cu") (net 26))
 (segment (start 145.77175 80.315) (end 144.56 81.52675) (width 0.25) (layer "F.Cu") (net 26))
 (segment (start 148.284864 77.775) (end 145.77175 77.775) (width 0.25) (layer "F.Cu") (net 27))
 (segment (start 145.77175 77.775) (end 144.56 78.98675) (width 0.25) (layer "F.Cu") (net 27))
 (segment (start 142.5 74.38675) (end 144.56 76.44675) (width 0.25) (layer "F.Cu") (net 28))
 (segment (start 142.5 72.65) (end 142.5 74.38675) (width 0.25) (layer "F.Cu") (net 28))
 (segment (start 148.284864 72.695) (end 148.239864 72.65) (width 0.25) (layer "F.Cu") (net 28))
 (segment (start 148.239864 72.65) (end 142.5 72.65) (width 0.25) (layer "F.Cu") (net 28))
 (segment (start 127.95496 103.175) (end 124.975 103.175) (width 0.25) (layer "F.Cu") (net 16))
 (via (at 124.975 103.175) (size 0.8) (drill 0.4) (layers "F.Cu" "B.Cu") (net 16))
 (segment (start 146.87 94.63) (end 146.87 76.21675) (width 0.25) (layer "B.Cu") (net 16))
 (segment (start 130.7 96.91) (end 144.59 96.91) (width 0.25) (layer "B.Cu") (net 16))
 (segment (start 124.975 103.175) (end 124.975 102.635) (width 0.25) (layer "B.Cu") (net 16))
 (segment (start 124.975 102.635) (end 130.7 96.91) (width 0.25) (layer "B.Cu") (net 16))
 (segment (start 144.59 96.91) (end 146.87 94.63) (width 0.25) (layer "B.Cu") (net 16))
 (segment (start 146.87 76.21675) (end 144.56 73.90675) (width 0.25) (layer "B.Cu") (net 16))
 (segment (start 148.284864 67.615) (end 148.284864 70.155) (width 0.25) (layer "F.Cu") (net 29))
 (segment (start 145.77175 70.155) (end 144.56 71.36675) (width 0.25) (layer "F.Cu") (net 29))
 (segment (start 148.284864 70.155) (end 145.77175 70.155) (width 0.25) (layer "F.Cu") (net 29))
 (segment (start 148.284864 82.855) (end 148.229864 82.8) (width 0.25) (layer "F.Cu") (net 25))
 (segment (start 140.85 72.53675) (end 144.56 68.82675) (width 0.25) (layer "F.Cu") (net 25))
 (segment (start 140.85 80.9) (end 140.85 72.53675) (width 0.25) (layer "F.Cu") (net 25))
 (segment (start 142.75 82.8) (end 140.85 80.9) (width 0.25) (layer "F.Cu") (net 25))
 (segment (start 148.229864 82.8) (end 142.75 82.8) (width 0.25) (layer "F.Cu") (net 25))
 (segment (start 142.25 59.55) (end 142.25 61.43675) (width 0.25) (layer "F.Cu") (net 32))
 (segment (start 142.25 61.43675) (end 144.56 63.74675) (width 0.25) (layer "F.Cu") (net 32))
 (segment (start 147.909864 57.455) (end 144.345 57.455) (width 0.25) (layer "F.Cu") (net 32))
 (segment (start 144.345 57.455) (end 142.25 59.55) (width 0.25) (layer "F.Cu") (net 32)))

